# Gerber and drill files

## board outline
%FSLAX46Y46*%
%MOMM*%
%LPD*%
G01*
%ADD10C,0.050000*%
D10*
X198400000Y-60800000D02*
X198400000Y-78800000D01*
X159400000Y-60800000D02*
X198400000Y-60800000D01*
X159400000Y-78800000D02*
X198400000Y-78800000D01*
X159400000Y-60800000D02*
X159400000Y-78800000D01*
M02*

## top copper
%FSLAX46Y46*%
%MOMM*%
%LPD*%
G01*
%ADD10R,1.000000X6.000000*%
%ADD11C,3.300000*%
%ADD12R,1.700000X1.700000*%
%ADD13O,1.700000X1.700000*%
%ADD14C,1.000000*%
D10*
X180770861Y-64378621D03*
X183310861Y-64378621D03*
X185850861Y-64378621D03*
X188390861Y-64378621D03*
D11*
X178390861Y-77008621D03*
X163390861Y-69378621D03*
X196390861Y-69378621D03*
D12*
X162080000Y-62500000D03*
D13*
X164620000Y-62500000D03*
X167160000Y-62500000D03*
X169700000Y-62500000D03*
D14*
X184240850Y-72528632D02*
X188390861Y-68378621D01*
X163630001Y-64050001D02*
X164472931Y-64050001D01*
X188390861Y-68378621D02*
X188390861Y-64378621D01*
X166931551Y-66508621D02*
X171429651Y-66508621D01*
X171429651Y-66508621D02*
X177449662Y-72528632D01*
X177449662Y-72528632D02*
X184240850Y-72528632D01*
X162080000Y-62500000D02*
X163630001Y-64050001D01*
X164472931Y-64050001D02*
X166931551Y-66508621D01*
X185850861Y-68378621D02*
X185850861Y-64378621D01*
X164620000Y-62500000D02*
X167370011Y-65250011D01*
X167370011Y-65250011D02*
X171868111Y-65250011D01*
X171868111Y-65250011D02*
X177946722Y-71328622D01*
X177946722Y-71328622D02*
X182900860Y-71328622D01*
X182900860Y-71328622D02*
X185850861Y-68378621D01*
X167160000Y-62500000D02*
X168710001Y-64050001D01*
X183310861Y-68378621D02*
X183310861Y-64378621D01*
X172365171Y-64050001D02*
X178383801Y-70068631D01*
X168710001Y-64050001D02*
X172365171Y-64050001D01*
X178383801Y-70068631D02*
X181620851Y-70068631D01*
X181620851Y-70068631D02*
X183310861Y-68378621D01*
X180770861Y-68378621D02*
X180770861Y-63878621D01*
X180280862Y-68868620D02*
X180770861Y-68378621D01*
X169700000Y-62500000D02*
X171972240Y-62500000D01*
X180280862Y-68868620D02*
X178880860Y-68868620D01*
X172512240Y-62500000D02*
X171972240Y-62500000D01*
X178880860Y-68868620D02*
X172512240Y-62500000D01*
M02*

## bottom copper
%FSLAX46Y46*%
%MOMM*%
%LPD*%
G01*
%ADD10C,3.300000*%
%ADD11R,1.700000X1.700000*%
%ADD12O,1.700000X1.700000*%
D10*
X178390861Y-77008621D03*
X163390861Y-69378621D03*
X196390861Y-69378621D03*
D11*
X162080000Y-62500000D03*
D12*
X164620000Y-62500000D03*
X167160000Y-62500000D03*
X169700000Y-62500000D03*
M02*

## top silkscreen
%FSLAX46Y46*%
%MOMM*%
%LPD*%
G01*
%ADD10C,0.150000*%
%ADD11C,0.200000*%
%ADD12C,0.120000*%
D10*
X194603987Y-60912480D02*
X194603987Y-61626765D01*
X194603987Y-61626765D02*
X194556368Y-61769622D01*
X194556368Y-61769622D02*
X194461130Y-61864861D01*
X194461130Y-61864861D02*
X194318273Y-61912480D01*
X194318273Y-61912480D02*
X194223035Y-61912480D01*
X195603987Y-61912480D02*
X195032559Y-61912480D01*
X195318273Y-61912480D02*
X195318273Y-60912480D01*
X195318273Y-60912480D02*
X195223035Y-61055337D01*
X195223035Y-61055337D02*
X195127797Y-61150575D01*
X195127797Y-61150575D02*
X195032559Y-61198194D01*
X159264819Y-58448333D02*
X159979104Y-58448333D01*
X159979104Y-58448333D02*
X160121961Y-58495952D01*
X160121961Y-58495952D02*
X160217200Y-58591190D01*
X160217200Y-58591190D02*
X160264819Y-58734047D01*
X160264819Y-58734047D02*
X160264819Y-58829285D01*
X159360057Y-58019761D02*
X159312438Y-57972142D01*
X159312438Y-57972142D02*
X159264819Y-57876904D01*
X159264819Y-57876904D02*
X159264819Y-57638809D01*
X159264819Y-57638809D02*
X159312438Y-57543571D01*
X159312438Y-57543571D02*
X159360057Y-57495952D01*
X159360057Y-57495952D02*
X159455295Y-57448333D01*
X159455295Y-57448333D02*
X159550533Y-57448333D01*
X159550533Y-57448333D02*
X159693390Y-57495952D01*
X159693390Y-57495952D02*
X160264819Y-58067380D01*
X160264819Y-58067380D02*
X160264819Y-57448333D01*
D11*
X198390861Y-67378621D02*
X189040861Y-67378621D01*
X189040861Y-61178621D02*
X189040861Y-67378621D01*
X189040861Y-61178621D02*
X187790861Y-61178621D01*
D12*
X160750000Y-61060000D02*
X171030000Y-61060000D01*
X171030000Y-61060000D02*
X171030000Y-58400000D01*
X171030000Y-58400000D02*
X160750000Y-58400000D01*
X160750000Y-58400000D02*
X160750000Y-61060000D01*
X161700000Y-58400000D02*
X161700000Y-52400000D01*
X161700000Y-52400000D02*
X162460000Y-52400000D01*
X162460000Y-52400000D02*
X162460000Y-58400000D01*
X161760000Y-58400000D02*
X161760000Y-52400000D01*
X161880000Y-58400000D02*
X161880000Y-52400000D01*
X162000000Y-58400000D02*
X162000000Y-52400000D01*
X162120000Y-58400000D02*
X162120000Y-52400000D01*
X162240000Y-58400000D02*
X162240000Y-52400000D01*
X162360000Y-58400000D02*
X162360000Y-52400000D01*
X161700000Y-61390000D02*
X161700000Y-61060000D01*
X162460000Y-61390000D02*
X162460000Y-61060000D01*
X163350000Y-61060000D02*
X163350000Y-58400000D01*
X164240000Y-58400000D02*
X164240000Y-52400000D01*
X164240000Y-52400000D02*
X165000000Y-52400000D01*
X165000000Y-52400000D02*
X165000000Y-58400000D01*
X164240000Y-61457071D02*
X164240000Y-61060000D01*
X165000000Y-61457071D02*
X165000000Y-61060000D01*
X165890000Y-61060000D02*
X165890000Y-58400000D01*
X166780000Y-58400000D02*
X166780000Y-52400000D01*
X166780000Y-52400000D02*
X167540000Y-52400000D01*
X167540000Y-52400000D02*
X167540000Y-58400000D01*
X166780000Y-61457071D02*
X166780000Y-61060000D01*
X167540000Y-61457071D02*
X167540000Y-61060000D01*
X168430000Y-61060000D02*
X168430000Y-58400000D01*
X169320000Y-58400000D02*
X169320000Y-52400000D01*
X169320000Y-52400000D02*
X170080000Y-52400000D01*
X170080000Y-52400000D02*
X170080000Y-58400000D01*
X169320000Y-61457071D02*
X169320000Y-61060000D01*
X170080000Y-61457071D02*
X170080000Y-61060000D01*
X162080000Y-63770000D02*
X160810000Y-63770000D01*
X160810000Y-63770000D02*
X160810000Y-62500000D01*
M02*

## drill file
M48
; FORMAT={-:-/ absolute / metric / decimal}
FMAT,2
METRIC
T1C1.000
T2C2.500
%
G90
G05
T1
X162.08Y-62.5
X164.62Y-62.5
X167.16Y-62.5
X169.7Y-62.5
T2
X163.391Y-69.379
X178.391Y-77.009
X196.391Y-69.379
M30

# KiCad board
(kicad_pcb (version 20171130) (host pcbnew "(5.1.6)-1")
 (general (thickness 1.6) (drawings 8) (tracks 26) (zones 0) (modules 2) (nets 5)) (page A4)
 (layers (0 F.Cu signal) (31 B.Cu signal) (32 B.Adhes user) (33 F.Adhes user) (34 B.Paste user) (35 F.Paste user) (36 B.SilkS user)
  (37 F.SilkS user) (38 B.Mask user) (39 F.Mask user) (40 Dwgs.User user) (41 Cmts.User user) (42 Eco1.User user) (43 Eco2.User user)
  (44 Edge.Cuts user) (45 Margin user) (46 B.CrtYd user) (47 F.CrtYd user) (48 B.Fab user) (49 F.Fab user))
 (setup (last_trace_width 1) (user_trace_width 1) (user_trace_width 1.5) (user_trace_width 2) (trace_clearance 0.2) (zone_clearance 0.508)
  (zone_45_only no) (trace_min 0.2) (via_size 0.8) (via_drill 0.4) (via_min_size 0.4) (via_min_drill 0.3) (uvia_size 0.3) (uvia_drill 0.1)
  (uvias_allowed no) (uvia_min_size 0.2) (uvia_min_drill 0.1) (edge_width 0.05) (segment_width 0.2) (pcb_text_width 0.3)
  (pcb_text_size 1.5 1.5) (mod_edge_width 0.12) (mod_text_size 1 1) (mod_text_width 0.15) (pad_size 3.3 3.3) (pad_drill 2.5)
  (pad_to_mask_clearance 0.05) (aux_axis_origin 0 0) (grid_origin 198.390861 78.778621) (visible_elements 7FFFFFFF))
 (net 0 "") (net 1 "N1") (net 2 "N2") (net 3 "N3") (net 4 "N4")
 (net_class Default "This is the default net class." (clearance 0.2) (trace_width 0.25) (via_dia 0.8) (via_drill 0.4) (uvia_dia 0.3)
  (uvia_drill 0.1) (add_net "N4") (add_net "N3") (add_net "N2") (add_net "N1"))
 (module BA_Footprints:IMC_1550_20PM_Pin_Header (layer F.Cu) (at 198.390861 67.378621)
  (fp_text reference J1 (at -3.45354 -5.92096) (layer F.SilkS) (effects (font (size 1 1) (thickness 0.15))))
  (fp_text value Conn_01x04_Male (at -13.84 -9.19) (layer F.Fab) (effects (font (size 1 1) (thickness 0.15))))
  (fp_line (start 0 0) (end -9.35 0) (layer F.SilkS) (width 0.2))
  (fp_line (start -9.35 -6.2) (end -9.35 0) (layer F.SilkS) (width 0.2))
  (fp_line (start -9.35 -6.2) (end -10.6 -6.2) (layer F.SilkS) (width 0.2))
  (pad 4 smd rect (at -17.62 -3) (size 1 6) (layers F.Cu F.Paste F.Mask) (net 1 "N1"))
  (pad 3 smd rect (at -15.08 -3) (size 1 6) (layers F.Cu F.Paste F.Mask) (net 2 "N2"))
  (pad 2 smd rect (at -12.54 -3) (size 1 6) (layers F.Cu F.Paste F.Mask) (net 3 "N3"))
  (pad 1 smd rect (at -10 -3) (size 1 6) (layers F.Cu F.Paste F.Mask) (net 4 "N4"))
  (pad "" np_thru_hole circle (at -20 9.63) (size 3.3 3.3) (drill 2.5) (layers *.Cu *.Mask))
  (pad "" np_thru_hole circle (at -35 2) (size 3.3 3.3) (drill 2.5) (layers *.Cu *.Mask))
  (pad "" np_thru_hole circle (at -2 2) (size 3.3 3.3) (drill 2.5) (layers *.Cu *.Mask)))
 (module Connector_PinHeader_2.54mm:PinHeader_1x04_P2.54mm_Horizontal (layer F.Cu) (at 162.08 62.5 90)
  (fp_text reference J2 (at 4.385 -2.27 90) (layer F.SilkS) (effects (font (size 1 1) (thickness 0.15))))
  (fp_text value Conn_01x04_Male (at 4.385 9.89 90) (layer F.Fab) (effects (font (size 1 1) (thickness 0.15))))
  (fp_line (start 1.44 -1.33) (end 1.44 8.95) (layer F.SilkS) (width 0.12))
  (fp_line (start 1.44 8.95) (end 4.1 8.95) (layer F.SilkS) (width 0.12))
  (fp_line (start 4.1 8.95) (end 4.1 -1.33) (layer F.SilkS) (width 0.12))
  (fp_line (start 4.1 -1.33) (end 1.44 -1.33) (layer F.SilkS) (width 0.12))
  (fp_line (start 4.1 -0.38) (end 10.1 -0.38) (layer F.SilkS) (width 0.12))
  (fp_line (start 10.1 -0.38) (end 10.1 0.38) (layer F.SilkS) (width 0.12))
  (fp_line (start 10.1 0.38) (end 4.1 0.38) (layer F.SilkS) (width 0.12))
  (fp_line (start 4.1 -0.32) (end 10.1 -0.32) (layer F.SilkS) (width 0.12))
  (fp_line (start 4.1 -0.2) (end 10.1 -0.2) (layer F.SilkS) (width 0.12))
  (fp_line (start 4.1 -0.08) (end 10.1 -0.08) (layer F.SilkS) (width 0.12))
  (fp_line (start 4.1 0.04) (end 10.1 0.04) (layer F.SilkS) (width 0.12))
  (fp_line (start 4.1 0.16) (end 10.1 0.16) (layer F.SilkS) (width 0.12))
  (fp_line (start 4.1 0.28) (end 10.1 0.28) (layer F.SilkS) (width 0.12))
  (fp_line (start 1.11 -0.38) (end 1.44 -0.38) (layer F.SilkS) (width 0.12))
  (fp_line (start 1.11 0.38) (end 1.44 0.38) (layer F.SilkS) (width 0.12))
  (fp_line (start 1.44 1.27) (end 4.1 1.27) (layer F.SilkS) (width 0.12))
  (fp_line (start 4.1 2.16) (end 10.1 2.16) (layer F.SilkS) (width 0.12))
  (fp_line (start 10.1 2.16) (end 10.1 2.92) (layer F.SilkS) (width 0.12))
  (fp_line (start 10.1 2.92) (end 4.1 2.92) (layer F.SilkS) (width 0.12))
  (fp_line (start 1.042929 2.16) (end 1.44 2.16) (layer F.SilkS) (width 0.12))
  (fp_line (start 1.042929 2.92) (end 1.44 2.92) (layer F.SilkS) (width 0.12))
  (fp_line (start 1.44 3.81) (end 4.1 3.81) (layer F.SilkS) (width 0.12))
  (fp_line (start 4.1 4.7) (end 10.1 4.7) (layer F.SilkS) (width 0.12))
  (fp_line (start 10.1 4.7) (end 10.1 5.46) (layer F.SilkS) (width 0.12))
  (fp_line (start 10.1 5.46) (end 4.1 5.46) (layer F.SilkS) (width 0.12))
  (fp_line (start 1.042929 4.7) (end 1.44 4.7) (layer F.SilkS) (width 0.12))
  (fp_line (start 1.042929 5.46) (end 1.44 5.46) (layer F.SilkS) (width 0.12))
  (fp_line (start 1.44 6.35) (end 4.1 6.35) (layer F.SilkS) (width 0.12))
  (fp_line (start 4.1 7.24) (end 10.1 7.24) (layer F.SilkS) (width 0.12))
  (fp_line (start 10.1 7.24) (end 10.1 8) (layer F.SilkS) (width 0.12))
  (fp_line (start 10.1 8) (end 4.1 8) (layer F.SilkS) (width 0.12))
  (fp_line (start 1.042929 7.24) (end 1.44 7.24) (layer F.SilkS) (width 0.12))
  (fp_line (start 1.042929 8) (end 1.44 8) (layer F.SilkS) (width 0.12))
  (fp_line (start -1.27 0) (end -1.27 -1.27) (layer F.SilkS) (width 0.12))
  (fp_line (start -1.27 -1.27) (end 0 -1.27) (layer F.SilkS) (width 0.12))
  (pad 1 thru_hole rect (at 0 0 90) (size 1.7 1.7) (drill 1) (layers *.Cu *.Mask) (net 4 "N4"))
  (pad 2 thru_hole oval (at 0 2.54 90) (size 1.7 1.7) (drill 1) (layers *.Cu *.Mask) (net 3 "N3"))
  (pad 3 thru_hole oval (at 0 5.08 90) (size 1.7 1.7) (drill 1) (layers *.Cu *.Mask) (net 2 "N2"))
  (pad 4 thru_hole oval (at 0 7.62 90) (size 1.7 1.7) (drill 1) (layers *.Cu *.Mask) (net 1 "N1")))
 (gr_line (start 198.4 60.8) (end 198.4 78.8) (layer Edge.Cuts) (width 0.05))
 (gr_line (start 159.4 60.8) (end 198.4 60.8) (layer Edge.Cuts) (width 0.05))
 (gr_line (start 159.4 78.8) (end 198.4 78.8) (layer Edge.Cuts) (width 0.05))
 (gr_line (start 159.4 60.8) (end 159.4 78.8) (layer Edge.Cuts) (width 0.05))
 (segment (start 184.24085 72.528632) (end 188.390861 68.378621) (width 1) (layer F.Cu) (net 4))
 (segment (start 163.630001 64.050001) (end 164.472931 64.050001) (width 1) (layer F.Cu) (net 4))
 (segment (start 188.390861 68.378621) (end 188.390861 64.378621) (width 1) (layer F.Cu) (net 4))
 (segment (start 166.931551 66.508621) (end 171.429651 66.508621) (width 1) (layer F.Cu) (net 4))
 (segment (start 171.429651 66.508621) (end 177.449662 72.528632) (width 1) (layer F.Cu) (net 4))
 (segment (start 177.449662 72.528632) (end 184.24085 72.528632) (width 1) (layer F.Cu) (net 4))
 (segment (start 162.08 62.5) (end 163.630001 64.050001) (width 1) (layer F.Cu) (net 4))
 (segment (start 164.472931 64.050001) (end 166.931551 66.508621) (width 1) (layer F.Cu) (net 4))
 (segment (start 185.850861 68.378621) (end 185.850861 64.378621) (width 1) (layer F.Cu) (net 3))
 (segment (start 164.62 62.5) (end 167.370011 65.250011) (width 1) (layer F.Cu) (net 3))
 (segment (start 167.370011 65.250011) (end 171.868111 65.250011) (width 1) (layer F.Cu) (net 3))
 (segment (start 171.868111 65.250011) (end 177.946722 71.328622) (width 1) (layer F.Cu) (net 3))
 (segment (start 177.946722 71.328622) (end 182.90086 71.328622) (width 1) (layer F.Cu) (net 3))
 (segment (start 182.90086 71.328622) (end 185.850861 68.378621) (width 1) (layer F.Cu) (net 3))
 (segment (start 167.16 62.5) (end 168.710001 64.050001) (width 1) (layer F.Cu) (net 2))
 (segment (start 183.310861 68.378621) (end 183.310861 64.378621) (width 1) (layer F.Cu) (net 2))
 (segment (start 172.365171 64.050001) (end 178.383801 70.068631) (width 1) (layer F.Cu) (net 2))
 (segment (start 168.710001 64.050001) (end 172.365171 64.050001) (width 1) (layer F.Cu) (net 2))
 (segment (start 178.383801 70.068631) (end 181.620851 70.068631) (width 1) (layer F.Cu) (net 2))
 (segment (start 181.620851 70.068631) (end 183.310861 68.378621) (width 1) (layer F.Cu) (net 2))
 (segment (start 180.770861 68.378621) (end 180.770861 63.878621) (width 1) (layer F.Cu) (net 1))
 (segment (start 180.280862 68.86862) (end 180.770861 68.378621) (width 1) (layer F.Cu) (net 1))
 (segment (start 169.7 62.5) (end 171.97224 62.5) (width 1) (layer F.Cu) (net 1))
 (segment (start 180.280862 68.86862) (end 178.88086 68.86862) (width 1) (layer F.Cu) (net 1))
 (segment (start 172.51224 62.5) (end 171.97224 62.5) (width 1) (layer F.Cu) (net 1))
 (segment (start 178.88086 68.86862) (end 172.51224 62.5) (width 1) (layer F.Cu) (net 1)))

